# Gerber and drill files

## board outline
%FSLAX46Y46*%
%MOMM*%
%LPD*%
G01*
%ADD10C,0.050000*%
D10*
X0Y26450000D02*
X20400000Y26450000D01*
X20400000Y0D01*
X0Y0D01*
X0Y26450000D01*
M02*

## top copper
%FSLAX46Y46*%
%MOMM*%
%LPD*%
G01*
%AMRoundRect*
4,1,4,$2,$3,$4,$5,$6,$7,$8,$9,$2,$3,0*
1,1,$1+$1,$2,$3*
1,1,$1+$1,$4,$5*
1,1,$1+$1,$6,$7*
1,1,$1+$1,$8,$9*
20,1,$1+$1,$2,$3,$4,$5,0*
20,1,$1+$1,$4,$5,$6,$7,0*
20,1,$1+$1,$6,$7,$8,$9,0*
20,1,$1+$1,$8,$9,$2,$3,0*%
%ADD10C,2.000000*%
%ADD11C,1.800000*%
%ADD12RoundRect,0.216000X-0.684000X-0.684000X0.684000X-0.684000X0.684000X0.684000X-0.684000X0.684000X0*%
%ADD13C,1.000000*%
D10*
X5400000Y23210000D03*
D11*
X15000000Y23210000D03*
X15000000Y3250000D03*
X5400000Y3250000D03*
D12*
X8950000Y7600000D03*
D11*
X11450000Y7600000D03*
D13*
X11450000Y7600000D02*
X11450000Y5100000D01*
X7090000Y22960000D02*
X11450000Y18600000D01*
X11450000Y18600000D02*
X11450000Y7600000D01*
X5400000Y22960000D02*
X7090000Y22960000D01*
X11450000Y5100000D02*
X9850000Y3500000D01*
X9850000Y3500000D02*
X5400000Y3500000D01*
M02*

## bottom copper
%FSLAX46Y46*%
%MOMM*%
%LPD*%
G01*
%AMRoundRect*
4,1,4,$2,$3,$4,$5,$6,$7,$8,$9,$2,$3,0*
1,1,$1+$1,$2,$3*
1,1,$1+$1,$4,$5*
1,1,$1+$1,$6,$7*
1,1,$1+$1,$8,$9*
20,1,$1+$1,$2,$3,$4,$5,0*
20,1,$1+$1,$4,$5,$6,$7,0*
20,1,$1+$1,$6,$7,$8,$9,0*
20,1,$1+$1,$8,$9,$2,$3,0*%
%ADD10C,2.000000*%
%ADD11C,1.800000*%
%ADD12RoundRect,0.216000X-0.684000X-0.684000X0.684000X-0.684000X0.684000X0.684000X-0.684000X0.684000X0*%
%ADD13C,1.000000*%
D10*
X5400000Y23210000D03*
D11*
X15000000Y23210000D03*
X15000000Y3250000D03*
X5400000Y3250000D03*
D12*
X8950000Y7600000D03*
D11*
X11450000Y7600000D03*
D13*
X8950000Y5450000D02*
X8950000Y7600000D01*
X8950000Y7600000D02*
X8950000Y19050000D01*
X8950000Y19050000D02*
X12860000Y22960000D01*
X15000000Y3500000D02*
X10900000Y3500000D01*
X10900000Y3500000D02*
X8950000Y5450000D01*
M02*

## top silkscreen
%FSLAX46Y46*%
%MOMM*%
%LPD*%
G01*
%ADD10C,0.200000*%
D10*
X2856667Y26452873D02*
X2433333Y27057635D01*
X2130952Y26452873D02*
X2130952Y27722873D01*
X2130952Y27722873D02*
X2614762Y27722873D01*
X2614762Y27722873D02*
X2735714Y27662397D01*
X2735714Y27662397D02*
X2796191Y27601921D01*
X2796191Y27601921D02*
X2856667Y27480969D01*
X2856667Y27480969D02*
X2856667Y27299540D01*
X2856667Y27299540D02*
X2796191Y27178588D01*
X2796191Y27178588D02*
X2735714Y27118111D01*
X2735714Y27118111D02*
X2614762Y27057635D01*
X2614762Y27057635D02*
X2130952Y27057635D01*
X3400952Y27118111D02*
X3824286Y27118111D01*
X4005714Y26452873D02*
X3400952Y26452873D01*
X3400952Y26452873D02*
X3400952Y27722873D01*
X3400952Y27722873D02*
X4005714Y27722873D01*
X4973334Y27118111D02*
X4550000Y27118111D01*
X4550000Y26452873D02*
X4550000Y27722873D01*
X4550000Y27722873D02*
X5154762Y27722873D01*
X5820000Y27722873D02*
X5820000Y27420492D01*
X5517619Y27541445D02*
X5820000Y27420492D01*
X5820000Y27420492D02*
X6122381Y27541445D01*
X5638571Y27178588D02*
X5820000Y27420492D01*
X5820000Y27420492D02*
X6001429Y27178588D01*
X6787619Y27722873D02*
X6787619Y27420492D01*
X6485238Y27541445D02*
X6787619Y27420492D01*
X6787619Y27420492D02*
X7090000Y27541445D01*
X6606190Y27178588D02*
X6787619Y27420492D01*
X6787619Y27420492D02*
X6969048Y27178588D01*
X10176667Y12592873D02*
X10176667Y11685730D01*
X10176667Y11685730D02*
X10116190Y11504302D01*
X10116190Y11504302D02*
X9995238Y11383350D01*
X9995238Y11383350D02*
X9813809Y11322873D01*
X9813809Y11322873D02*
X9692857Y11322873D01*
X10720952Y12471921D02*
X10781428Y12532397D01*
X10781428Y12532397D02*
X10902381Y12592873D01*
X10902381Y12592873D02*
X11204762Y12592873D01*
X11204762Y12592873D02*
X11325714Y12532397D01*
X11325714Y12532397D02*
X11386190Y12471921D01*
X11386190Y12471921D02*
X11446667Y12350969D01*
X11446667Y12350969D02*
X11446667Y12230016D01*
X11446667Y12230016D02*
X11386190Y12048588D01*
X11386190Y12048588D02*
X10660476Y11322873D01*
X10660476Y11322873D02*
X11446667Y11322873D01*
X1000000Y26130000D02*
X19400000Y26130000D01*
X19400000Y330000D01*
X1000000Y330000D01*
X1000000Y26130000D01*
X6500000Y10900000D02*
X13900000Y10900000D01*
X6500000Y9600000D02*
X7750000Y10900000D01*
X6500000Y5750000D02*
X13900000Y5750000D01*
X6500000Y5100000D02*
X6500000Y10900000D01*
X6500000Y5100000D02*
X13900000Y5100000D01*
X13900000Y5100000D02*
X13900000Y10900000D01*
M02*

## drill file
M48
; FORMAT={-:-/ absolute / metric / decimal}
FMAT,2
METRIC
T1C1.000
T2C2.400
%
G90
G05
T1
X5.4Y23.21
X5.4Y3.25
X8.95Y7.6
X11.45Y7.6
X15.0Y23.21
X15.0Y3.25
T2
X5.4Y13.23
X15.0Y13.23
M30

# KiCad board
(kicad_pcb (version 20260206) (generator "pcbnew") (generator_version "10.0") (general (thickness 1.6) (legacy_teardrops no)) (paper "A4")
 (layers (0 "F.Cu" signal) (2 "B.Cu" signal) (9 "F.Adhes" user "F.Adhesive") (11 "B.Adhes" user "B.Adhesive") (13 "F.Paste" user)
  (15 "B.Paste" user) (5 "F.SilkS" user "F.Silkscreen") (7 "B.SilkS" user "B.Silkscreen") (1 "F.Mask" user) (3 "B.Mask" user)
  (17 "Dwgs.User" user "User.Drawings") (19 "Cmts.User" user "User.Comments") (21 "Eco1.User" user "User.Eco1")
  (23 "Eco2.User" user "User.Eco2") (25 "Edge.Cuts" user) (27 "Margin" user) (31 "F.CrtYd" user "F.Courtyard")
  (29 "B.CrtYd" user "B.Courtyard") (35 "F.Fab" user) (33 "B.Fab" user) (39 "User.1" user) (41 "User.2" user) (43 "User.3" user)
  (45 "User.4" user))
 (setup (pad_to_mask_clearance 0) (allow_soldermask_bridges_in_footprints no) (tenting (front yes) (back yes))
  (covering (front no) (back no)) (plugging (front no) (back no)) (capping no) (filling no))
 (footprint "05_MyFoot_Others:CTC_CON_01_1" (layer "F.Cu") (at 10.2 -13.23)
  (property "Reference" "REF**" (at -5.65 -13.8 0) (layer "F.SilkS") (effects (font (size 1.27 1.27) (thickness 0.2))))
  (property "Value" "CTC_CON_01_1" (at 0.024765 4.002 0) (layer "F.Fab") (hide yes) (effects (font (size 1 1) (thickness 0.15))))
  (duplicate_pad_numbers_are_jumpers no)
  (fp_rect (start -9.2 -12.9) (end 9.2 12.9) (stroke (width 0.2) (type default)) (fill no) (layer "F.SilkS"))
  (pad "" np_thru_hole circle (at -4.8 0) (size 2.4 2.4) (drill 2.4) (layers "*.Cu") (thermal_bridge_angle 90))
  (pad "" np_thru_hole circle (at 4.8 0) (size 2.4 2.4) (drill 2.4) (layers "*.Cu") (thermal_bridge_angle 90))
  (pad "1" thru_hole circle (at -4.8 -9.98) (size 2 2) (drill 1) (layers "*.Cu" "*.Mask") (remove_unused_layers no))
  (pad "2" thru_hole circle (at 4.8 -9.98) (size 1.8 1.8) (drill 1) (layers "*.Cu" "*.Mask") (remove_unused_layers no)
   (thermal_bridge_angle 90))
  (pad "3" thru_hole circle (at 4.8 9.98) (size 1.8 1.8) (drill 1) (layers "*.Cu" "*.Mask") (remove_unused_layers no)
   (thermal_bridge_angle 90))
  (pad "4" thru_hole circle (at -4.8 9.98) (size 1.8 1.8) (drill 1) (layers "*.Cu" "*.Mask") (remove_unused_layers no)
   (thermal_bridge_angle 90)))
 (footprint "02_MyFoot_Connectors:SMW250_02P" (layer "F.Cu") (at 10.2 -7.6)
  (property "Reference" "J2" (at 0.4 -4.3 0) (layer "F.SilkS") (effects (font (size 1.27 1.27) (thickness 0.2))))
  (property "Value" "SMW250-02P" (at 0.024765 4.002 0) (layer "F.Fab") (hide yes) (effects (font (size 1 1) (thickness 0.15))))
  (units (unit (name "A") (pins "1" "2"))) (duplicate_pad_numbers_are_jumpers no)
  (fp_line (start -3.7 -3.3) (end 3.7 -3.3) (stroke (width 0.2) (type solid)) (layer "F.SilkS"))
  (fp_line (start -3.7 -2) (end -2.45 -3.3) (stroke (width 0.2) (type solid)) (layer "F.SilkS"))
  (fp_line (start -3.7 1.85) (end 3.7 1.85) (stroke (width 0.2) (type solid)) (layer "F.SilkS"))
  (fp_line (start -3.7 2.5) (end -3.7 -3.3) (stroke (width 0.2) (type solid)) (layer "F.SilkS"))
  (fp_line (start -3.7 2.5) (end 3.7 2.5) (stroke (width 0.2) (type solid)) (layer "F.SilkS"))
  (fp_line (start 3.7 2.5) (end 3.7 -3.3) (stroke (width 0.2) (type solid)) (layer "F.SilkS"))
  (pad "1" thru_hole roundrect (at -1.25 0) (size 1.8 1.8) (drill 1) (layers "*.Cu" "*.Mask") (remove_unused_layers no)
   (roundrect_rratio 0.12) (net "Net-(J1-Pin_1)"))
  (pad "2" thru_hole circle (at 1.25 0) (size 1.8 1.8) (drill 1) (layers "*.Cu" "*.Mask") (remove_unused_layers no) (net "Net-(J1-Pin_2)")
   (thermal_bridge_angle 90)))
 (gr_rect (start 0 -26.45) (end 20.4 0) (stroke (width 0.05) (type solid)) (fill no) (layer "Edge.Cuts"))
 (segment (start 8.95 -5.45) (end 8.95 -7.6) (width 1) (layer "B.Cu") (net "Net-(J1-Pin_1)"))
 (segment (start 8.95 -7.6) (end 8.95 -19.05) (width 1) (layer "B.Cu") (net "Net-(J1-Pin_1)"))
 (segment (start 8.95 -19.05) (end 12.86 -22.96) (width 1) (layer "B.Cu") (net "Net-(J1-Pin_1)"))
 (segment (start 15 -3.5) (end 10.9 -3.5) (width 1) (layer "B.Cu") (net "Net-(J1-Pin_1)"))
 (segment (start 10.9 -3.5) (end 8.95 -5.45) (width 1) (layer "B.Cu") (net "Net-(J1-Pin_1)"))
 (segment (start 11.45 -7.6) (end 11.45 -5.1) (width 1) (layer "F.Cu") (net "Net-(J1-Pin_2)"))
 (segment (start 7.09 -22.96) (end 11.45 -18.6) (width 1) (layer "F.Cu") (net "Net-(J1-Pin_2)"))
 (segment (start 11.45 -18.6) (end 11.45 -7.6) (width 1) (layer "F.Cu") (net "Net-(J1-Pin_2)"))
 (segment (start 5.4 -22.96) (end 7.09 -22.96) (width 1) (layer "F.Cu") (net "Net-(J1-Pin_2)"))
 (segment (start 11.45 -5.1) (end 9.85 -3.5) (width 1) (layer "F.Cu") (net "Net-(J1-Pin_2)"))
 (segment (start 9.85 -3.5) (end 5.4 -3.5) (width 1) (layer "F.Cu") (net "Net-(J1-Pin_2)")))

